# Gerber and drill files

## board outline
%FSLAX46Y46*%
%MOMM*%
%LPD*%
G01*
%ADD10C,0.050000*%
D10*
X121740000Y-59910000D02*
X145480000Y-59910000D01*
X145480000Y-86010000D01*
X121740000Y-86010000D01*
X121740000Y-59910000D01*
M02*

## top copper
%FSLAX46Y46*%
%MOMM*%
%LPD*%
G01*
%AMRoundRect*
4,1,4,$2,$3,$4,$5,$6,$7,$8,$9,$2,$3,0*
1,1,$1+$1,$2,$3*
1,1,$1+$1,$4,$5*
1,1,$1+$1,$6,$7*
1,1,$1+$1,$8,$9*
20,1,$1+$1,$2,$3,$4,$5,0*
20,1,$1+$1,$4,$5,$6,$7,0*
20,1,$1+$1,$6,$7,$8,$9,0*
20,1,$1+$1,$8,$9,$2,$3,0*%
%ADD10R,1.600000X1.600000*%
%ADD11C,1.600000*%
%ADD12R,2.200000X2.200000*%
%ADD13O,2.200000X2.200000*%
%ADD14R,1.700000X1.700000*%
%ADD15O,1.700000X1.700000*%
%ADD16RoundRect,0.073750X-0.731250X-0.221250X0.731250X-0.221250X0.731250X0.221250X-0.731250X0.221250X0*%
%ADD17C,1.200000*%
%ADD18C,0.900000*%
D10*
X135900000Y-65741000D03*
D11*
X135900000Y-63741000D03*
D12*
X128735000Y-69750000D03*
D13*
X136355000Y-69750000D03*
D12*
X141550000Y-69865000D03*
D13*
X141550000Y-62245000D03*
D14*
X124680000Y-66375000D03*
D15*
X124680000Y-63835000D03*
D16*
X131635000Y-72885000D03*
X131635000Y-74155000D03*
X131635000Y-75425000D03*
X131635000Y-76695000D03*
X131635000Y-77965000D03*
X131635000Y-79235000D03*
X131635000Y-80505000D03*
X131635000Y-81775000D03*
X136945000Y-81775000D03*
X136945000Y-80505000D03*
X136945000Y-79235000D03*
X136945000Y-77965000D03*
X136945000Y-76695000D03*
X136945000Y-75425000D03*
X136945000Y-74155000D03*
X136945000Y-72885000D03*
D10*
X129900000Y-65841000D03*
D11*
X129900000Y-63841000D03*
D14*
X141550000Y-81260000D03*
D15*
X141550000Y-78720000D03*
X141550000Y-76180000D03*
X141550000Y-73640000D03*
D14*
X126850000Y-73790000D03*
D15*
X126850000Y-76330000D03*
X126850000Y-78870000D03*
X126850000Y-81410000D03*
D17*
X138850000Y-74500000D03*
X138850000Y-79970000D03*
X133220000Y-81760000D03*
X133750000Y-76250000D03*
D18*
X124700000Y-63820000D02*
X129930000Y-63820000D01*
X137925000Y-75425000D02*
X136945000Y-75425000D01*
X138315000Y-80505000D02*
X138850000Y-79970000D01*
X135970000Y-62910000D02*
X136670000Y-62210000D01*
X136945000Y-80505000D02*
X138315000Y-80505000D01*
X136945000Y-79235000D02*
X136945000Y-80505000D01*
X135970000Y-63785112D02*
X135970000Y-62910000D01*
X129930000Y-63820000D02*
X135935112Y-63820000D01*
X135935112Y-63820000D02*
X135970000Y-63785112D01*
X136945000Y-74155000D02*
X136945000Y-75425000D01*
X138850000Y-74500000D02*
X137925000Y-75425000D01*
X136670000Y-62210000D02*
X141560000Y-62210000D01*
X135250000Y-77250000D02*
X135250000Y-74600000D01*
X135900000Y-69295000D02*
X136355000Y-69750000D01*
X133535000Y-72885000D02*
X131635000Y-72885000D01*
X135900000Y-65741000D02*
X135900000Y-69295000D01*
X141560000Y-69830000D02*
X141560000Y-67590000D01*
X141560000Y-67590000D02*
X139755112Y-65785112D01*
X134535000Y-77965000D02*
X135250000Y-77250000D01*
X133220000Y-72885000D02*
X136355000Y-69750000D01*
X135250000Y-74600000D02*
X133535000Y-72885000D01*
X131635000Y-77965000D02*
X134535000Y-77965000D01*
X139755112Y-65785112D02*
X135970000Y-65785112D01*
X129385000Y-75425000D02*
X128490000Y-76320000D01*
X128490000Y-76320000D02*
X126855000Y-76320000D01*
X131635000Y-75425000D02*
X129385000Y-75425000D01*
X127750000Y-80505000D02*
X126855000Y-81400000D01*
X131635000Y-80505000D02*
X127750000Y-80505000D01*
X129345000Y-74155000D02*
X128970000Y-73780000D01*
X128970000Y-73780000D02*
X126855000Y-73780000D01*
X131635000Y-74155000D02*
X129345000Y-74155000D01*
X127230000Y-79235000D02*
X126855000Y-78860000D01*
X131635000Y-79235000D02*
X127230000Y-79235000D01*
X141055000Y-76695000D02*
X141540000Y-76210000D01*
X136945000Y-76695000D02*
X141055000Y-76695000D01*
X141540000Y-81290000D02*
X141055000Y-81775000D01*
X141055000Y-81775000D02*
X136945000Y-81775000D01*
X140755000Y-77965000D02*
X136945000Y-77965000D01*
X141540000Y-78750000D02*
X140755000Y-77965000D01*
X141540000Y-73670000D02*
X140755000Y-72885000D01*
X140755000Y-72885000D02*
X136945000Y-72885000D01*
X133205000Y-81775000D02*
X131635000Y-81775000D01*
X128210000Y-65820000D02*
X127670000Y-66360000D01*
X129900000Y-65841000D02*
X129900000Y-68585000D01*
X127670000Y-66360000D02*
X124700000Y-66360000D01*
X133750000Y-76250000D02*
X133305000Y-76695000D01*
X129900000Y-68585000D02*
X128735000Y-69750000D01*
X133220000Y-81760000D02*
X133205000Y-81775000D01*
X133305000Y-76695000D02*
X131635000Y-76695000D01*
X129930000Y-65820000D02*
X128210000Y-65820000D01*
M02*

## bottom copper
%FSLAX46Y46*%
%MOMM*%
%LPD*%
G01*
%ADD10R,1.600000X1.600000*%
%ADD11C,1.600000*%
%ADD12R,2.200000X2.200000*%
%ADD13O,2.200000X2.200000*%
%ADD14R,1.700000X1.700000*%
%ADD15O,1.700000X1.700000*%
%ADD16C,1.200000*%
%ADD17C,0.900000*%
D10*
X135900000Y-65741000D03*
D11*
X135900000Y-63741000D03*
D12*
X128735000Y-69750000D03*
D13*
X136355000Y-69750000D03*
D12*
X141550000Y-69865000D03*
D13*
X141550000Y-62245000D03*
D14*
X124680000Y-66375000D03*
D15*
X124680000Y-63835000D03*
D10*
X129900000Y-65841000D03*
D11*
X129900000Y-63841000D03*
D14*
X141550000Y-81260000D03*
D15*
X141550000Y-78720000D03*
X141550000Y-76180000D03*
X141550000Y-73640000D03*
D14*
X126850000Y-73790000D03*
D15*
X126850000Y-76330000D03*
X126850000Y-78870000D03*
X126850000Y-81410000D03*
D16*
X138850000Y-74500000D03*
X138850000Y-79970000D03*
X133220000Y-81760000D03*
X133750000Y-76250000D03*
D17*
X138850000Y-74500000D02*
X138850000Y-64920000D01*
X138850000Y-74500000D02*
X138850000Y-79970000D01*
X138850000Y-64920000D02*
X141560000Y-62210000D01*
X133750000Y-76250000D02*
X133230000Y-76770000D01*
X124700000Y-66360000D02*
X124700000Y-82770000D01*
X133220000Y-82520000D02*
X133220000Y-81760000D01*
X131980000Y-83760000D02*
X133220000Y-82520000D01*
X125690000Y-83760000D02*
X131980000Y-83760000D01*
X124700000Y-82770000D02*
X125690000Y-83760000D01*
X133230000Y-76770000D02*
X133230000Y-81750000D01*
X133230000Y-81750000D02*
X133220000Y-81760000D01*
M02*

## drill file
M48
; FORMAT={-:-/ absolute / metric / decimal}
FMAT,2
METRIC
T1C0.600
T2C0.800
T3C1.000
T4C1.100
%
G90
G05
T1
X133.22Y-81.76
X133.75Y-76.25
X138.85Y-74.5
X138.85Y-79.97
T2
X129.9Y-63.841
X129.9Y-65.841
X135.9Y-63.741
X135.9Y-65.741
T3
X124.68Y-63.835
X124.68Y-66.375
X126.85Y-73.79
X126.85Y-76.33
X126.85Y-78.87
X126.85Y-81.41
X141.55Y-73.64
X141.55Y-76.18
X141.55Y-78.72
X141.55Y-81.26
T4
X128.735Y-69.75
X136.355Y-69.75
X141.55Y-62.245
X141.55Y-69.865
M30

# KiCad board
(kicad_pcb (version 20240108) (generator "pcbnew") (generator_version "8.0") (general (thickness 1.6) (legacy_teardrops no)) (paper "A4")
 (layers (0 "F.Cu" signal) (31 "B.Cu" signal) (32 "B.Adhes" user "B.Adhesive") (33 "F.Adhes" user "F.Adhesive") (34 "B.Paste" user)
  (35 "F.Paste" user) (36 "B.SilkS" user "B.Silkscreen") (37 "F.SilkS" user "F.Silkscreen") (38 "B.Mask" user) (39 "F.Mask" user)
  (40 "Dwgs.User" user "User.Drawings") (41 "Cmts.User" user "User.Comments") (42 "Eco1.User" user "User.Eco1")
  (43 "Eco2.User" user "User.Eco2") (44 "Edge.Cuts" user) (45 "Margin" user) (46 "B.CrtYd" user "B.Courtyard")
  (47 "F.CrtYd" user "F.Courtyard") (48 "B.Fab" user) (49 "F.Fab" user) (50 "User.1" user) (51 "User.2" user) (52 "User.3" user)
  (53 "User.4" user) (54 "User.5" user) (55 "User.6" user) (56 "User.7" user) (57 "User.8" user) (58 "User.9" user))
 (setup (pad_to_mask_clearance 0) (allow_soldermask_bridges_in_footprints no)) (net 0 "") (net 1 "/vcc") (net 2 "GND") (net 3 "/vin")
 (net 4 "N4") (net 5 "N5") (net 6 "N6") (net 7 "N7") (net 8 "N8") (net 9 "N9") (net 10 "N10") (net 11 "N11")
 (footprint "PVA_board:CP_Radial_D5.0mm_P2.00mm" (layer "F.Cu") (at 135.9 64.7 90)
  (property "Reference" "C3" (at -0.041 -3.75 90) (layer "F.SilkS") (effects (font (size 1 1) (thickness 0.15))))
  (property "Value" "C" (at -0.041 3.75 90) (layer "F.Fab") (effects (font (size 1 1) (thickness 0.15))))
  (pad "1" thru_hole rect (at -1.041 0 90) (size 1.6 1.6) (drill 0.8) (layers "*.Cu" "*.Mask") (remove_unused_layers no) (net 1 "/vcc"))
  (pad "2" thru_hole circle (at 0.959 0 90) (size 1.6 1.6) (drill 0.8) (layers "*.Cu" "*.Mask") (remove_unused_layers no) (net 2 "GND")))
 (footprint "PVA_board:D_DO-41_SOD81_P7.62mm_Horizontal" (layer "F.Cu") (at 132.5 69.75)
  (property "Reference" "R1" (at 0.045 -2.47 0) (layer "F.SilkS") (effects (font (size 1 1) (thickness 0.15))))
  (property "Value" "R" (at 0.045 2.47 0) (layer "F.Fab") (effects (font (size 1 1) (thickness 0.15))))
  (pad "1" thru_hole rect (at -3.765 0) (size 2.2 2.2) (drill 1.1) (layers "*.Cu" "*.Mask") (remove_unused_layers no) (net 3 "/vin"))
  (pad "2" thru_hole oval (at 3.855 0) (size 2.2 2.2) (drill 1.1) (layers "*.Cu" "*.Mask") (remove_unused_layers no) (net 1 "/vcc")))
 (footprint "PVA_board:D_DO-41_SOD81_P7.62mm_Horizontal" (layer "F.Cu") (at 141.55 66.1 90)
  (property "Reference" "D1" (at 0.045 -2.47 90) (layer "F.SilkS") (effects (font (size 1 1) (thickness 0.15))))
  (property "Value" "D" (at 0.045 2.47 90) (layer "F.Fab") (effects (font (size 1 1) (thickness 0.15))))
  (pad "1" thru_hole rect (at -3.765 0 90) (size 2.2 2.2) (drill 1.1) (layers "*.Cu" "*.Mask") (remove_unused_layers no) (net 1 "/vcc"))
  (pad "2" thru_hole oval (at 3.855 0 90) (size 2.2 2.2) (drill 1.1) (layers "*.Cu" "*.Mask") (remove_unused_layers no) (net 2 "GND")))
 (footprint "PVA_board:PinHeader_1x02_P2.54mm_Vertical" (layer "F.Cu") (at 124.6 65.055 180)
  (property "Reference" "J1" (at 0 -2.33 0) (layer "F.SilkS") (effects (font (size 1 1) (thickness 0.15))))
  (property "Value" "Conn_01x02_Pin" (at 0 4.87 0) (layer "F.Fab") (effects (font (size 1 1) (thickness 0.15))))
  (pad "1" thru_hole rect (at -0.08 -1.32 180) (size 1.7 1.7) (drill 1) (layers "*.Cu" "*.Mask") (remove_unused_layers no) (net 3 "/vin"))
  (pad "2" thru_hole oval (at -0.08 1.22 180) (size 1.7 1.7) (drill 1) (layers "*.Cu" "*.Mask") (remove_unused_layers no) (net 2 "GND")))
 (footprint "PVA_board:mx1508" (layer "F.Cu") (at 134.29 77.33)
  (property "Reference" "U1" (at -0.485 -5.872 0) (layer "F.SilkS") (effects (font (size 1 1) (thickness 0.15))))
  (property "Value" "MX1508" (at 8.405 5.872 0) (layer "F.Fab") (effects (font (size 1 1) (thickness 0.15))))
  (pad "1" smd roundrect (at -2.655 -4.445) (size 1.61 0.59) (layers "F.Cu" "F.Paste" "F.Mask") (roundrect_rratio 0.125) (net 1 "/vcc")
   (solder_mask_margin 0.102))
  (pad "2" smd roundrect (at -2.655 -3.175) (size 1.61 0.59) (layers "F.Cu" "F.Paste" "F.Mask") (roundrect_rratio 0.125) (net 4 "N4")
   (solder_mask_margin 0.102))
  (pad "3" smd roundrect (at -2.655 -1.905) (size 1.61 0.59) (layers "F.Cu" "F.Paste" "F.Mask") (roundrect_rratio 0.125) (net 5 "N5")
   (solder_mask_margin 0.102))
  (pad "4" smd roundrect (at -2.655 -0.635) (size 1.61 0.59) (layers "F.Cu" "F.Paste" "F.Mask") (roundrect_rratio 0.125) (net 3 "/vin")
   (solder_mask_margin 0.102))
  (pad "5" smd roundrect (at -2.655 0.635) (size 1.61 0.59) (layers "F.Cu" "F.Paste" "F.Mask") (roundrect_rratio 0.125) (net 1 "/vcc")
   (solder_mask_margin 0.102))
  (pad "6" smd roundrect (at -2.655 1.905) (size 1.61 0.59) (layers "F.Cu" "F.Paste" "F.Mask") (roundrect_rratio 0.125) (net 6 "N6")
   (solder_mask_margin 0.102))
  (pad "7" smd roundrect (at -2.655 3.175) (size 1.61 0.59) (layers "F.Cu" "F.Paste" "F.Mask") (roundrect_rratio 0.125) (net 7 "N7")
   (solder_mask_margin 0.102))
  (pad "8" smd roundrect (at -2.655 4.445) (size 1.61 0.59) (layers "F.Cu" "F.Paste" "F.Mask") (roundrect_rratio 0.125) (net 3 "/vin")
   (solder_mask_margin 0.102))
  (pad "9" smd roundrect (at 2.655 4.445) (size 1.61 0.59) (layers "F.Cu" "F.Paste" "F.Mask") (roundrect_rratio 0.125) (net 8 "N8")
   (solder_mask_margin 0.102))
  (pad "10" smd roundrect (at 2.655 3.175) (size 1.61 0.59) (layers "F.Cu" "F.Paste" "F.Mask") (roundrect_rratio 0.125) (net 2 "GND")
   (solder_mask_margin 0.102))
  (pad "11" smd roundrect (at 2.655 1.905) (size 1.61 0.59) (layers "F.Cu" "F.Paste" "F.Mask") (roundrect_rratio 0.125) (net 2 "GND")
   (solder_mask_margin 0.102))
  (pad "12" smd roundrect (at 2.655 0.635) (size 1.61 0.59) (layers "F.Cu" "F.Paste" "F.Mask") (roundrect_rratio 0.125) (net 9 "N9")
   (solder_mask_margin 0.102))
  (pad "13" smd roundrect (at 2.655 -0.635) (size 1.61 0.59) (layers "F.Cu" "F.Paste" "F.Mask") (roundrect_rratio 0.125) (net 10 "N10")
   (solder_mask_margin 0.102))
  (pad "14" smd roundrect (at 2.655 -1.905) (size 1.61 0.59) (layers "F.Cu" "F.Paste" "F.Mask") (roundrect_rratio 0.125) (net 2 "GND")
   (solder_mask_margin 0.102))
  (pad "15" smd roundrect (at 2.655 -3.175) (size 1.61 0.59) (layers "F.Cu" "F.Paste" "F.Mask") (roundrect_rratio 0.125) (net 2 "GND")
   (solder_mask_margin 0.102))
  (pad "16" smd roundrect (at 2.655 -4.445) (size 1.61 0.59) (layers "F.Cu" "F.Paste" "F.Mask") (roundrect_rratio 0.125) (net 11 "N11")
   (solder_mask_margin 0.102)))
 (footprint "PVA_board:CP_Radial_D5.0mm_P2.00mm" (layer "F.Cu") (at 129.9 64.8 90)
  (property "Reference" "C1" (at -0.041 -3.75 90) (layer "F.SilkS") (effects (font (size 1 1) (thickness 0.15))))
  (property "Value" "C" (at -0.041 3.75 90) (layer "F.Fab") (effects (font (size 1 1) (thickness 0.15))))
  (pad "1" thru_hole rect (at -1.041 0 90) (size 1.6 1.6) (drill 0.8) (layers "*.Cu" "*.Mask") (remove_unused_layers no) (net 3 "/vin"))
  (pad "2" thru_hole circle (at 0.959 0 90) (size 1.6 1.6) (drill 0.8) (layers "*.Cu" "*.Mask") (remove_unused_layers no) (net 2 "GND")))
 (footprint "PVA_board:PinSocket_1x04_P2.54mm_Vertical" (layer "F.Cu") (at 141.55 77.4 180)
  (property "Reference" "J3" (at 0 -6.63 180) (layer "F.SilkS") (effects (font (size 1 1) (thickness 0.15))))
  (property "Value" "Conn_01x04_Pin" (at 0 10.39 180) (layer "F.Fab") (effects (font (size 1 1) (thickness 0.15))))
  (pad "1" thru_hole rect (at 0 -3.86 180) (size 1.7 1.7) (drill 1) (layers "*.Cu" "*.Mask") (remove_unused_layers no) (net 8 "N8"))
  (pad "2" thru_hole oval (at 0 -1.32 180) (size 1.7 1.7) (drill 1) (layers "*.Cu" "*.Mask") (remove_unused_layers no) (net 9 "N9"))
  (pad "3" thru_hole oval (at 0 1.22 180) (size 1.7 1.7) (drill 1) (layers "*.Cu" "*.Mask") (remove_unused_layers no) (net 10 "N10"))
  (pad "4" thru_hole oval (at 0 3.76 180) (size 1.7 1.7) (drill 1) (layers "*.Cu" "*.Mask") (remove_unused_layers no) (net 11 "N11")))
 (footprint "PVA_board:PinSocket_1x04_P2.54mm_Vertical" (layer "F.Cu") (at 126.85 77.65)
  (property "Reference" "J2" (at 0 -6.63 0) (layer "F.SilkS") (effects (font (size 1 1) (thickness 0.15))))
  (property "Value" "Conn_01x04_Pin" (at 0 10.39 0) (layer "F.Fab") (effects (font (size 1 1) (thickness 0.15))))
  (pad "1" thru_hole rect (at 0 -3.86) (size 1.7 1.7) (drill 1) (layers "*.Cu" "*.Mask") (remove_unused_layers no) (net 4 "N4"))
  (pad "2" thru_hole oval (at 0 -1.32) (size 1.7 1.7) (drill 1) (layers "*.Cu" "*.Mask") (remove_unused_layers no) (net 5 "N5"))
  (pad "3" thru_hole oval (at 0 1.22) (size 1.7 1.7) (drill 1) (layers "*.Cu" "*.Mask") (remove_unused_layers no) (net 6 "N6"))
  (pad "4" thru_hole oval (at 0 3.76) (size 1.7 1.7) (drill 1) (layers "*.Cu" "*.Mask") (remove_unused_layers no) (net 7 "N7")))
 (gr_rect (start 121.74 59.91) (end 145.48 86.01) (stroke (width 0.05) (type default)) (fill none) (layer "Edge.Cuts"))
 (segment (start 124.7 63.82) (end 129.93 63.82) (width 0.9) (layer "F.Cu") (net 2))
 (segment (start 137.925 75.425) (end 136.945 75.425) (width 0.9) (layer "F.Cu") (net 2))
 (segment (start 138.315 80.505) (end 138.85 79.97) (width 0.9) (layer "F.Cu") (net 2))
 (segment (start 135.97 62.91) (end 136.67 62.21) (width 0.9) (layer "F.Cu") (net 2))
 (segment (start 136.945 80.505) (end 138.315 80.505) (width 0.9) (layer "F.Cu") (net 2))
 (segment (start 136.945 79.235) (end 136.945 80.505) (width 0.9) (layer "F.Cu") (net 2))
 (segment (start 135.97 63.785112) (end 135.97 62.91) (width 0.9) (layer "F.Cu") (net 2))
 (segment (start 129.93 63.82) (end 135.935112 63.82) (width 0.9) (layer "F.Cu") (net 2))
 (segment (start 135.935112 63.82) (end 135.97 63.785112) (width 0.9) (layer "F.Cu") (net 2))
 (segment (start 136.945 74.155) (end 136.945 75.425) (width 0.9) (layer "F.Cu") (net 2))
 (segment (start 138.85 74.5) (end 137.925 75.425) (width 0.9) (layer "F.Cu") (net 2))
 (segment (start 136.67 62.21) (end 141.56 62.21) (width 0.9) (layer "F.Cu") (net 2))
 (via (at 138.85 74.5) (size 1.2) (drill 0.6) (layers "F.Cu" "B.Cu") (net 2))
 (via (at 138.85 79.97) (size 1.2) (drill 0.6) (layers "F.Cu" "B.Cu") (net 2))
 (segment (start 138.85 74.5) (end 138.85 64.92) (width 0.9) (layer "B.Cu") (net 2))
 (segment (start 138.85 74.5) (end 138.85 79.97) (width 0.9) (layer "B.Cu") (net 2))
 (segment (start 138.85 64.92) (end 141.56 62.21) (width 0.9) (layer "B.Cu") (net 2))
 (segment (start 135.25 77.25) (end 135.25 74.6) (width 0.9) (layer "F.Cu") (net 1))
 (segment (start 135.9 69.295) (end 136.355 69.75) (width 0.9) (layer "F.Cu") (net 1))
 (segment (start 133.535 72.885) (end 131.635 72.885) (width 0.9) (layer "F.Cu") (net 1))
 (segment (start 135.9 65.741) (end 135.9 69.295) (width 0.9) (layer "F.Cu") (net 1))
 (segment (start 141.56 69.83) (end 141.56 67.59) (width 0.9) (layer "F.Cu") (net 1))
 (segment (start 141.56 67.59) (end 139.755112 65.785112) (width 0.9) (layer "F.Cu") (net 1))
 (segment (start 134.535 77.965) (end 135.25 77.25) (width 0.9) (layer "F.Cu") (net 1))
 (segment (start 133.22 72.885) (end 136.355 69.75) (width 0.9) (layer "F.Cu") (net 1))
 (segment (start 135.25 74.6) (end 133.535 72.885) (width 0.9) (layer "F.Cu") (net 1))
 (segment (start 131.635 77.965) (end 134.535 77.965) (width 0.9) (layer "F.Cu") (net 1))
 (segment (start 139.755112 65.785112) (end 135.97 65.785112) (width 0.9) (layer "F.Cu") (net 1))
 (segment (start 129.385 75.425) (end 128.49 76.32) (width 0.9) (layer "F.Cu") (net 5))
 (segment (start 128.49 76.32) (end 126.855 76.32) (width 0.9) (layer "F.Cu") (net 5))
 (segment (start 131.635 75.425) (end 129.385 75.425) (width 0.9) (layer "F.Cu") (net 5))
 (segment (start 127.75 80.505) (end 126.855 81.4) (width 0.9) (layer "F.Cu") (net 7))
 (segment (start 131.635 80.505) (end 127.75 80.505) (width 0.9) (layer "F.Cu") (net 7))
 (segment (start 129.345 74.155) (end 128.97 73.78) (width 0.9) (layer "F.Cu") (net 4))
 (segment (start 128.97 73.78) (end 126.855 73.78) (width 0.9) (layer "F.Cu") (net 4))
 (segment (start 131.635 74.155) (end 129.345 74.155) (width 0.9) (layer "F.Cu") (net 4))
 (segment (start 127.23 79.235) (end 126.855 78.86) (width 0.9) (layer "F.Cu") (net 6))
 (segment (start 131.635 79.235) (end 127.23 79.235) (width 0.9) (layer "F.Cu") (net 6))
 (segment (start 141.055 76.695) (end 141.54 76.21) (width 0.9) (layer "F.Cu") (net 10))
 (segment (start 136.945 76.695) (end 141.055 76.695) (width 0.9) (layer "F.Cu") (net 10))
 (segment (start 141.54 81.29) (end 141.055 81.775) (width 0.9) (layer "F.Cu") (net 8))
 (segment (start 141.055 81.775) (end 136.945 81.775) (width 0.9) (layer "F.Cu") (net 8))
 (segment (start 140.755 77.965) (end 136.945 77.965) (width 0.9) (layer "F.Cu") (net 9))
 (segment (start 141.54 78.75) (end 140.755 77.965) (width 0.9) (layer "F.Cu") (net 9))
 (segment (start 141.54 73.67) (end 140.755 72.885) (width 0.9) (layer "F.Cu") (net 11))
 (segment (start 140.755 72.885) (end 136.945 72.885) (width 0.9) (layer "F.Cu") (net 11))
 (segment (start 133.205 81.775) (end 131.635 81.775) (width 0.9) (layer "F.Cu") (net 3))
 (segment (start 128.21 65.82) (end 127.67 66.36) (width 0.9) (layer "F.Cu") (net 3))
 (segment (start 129.9 65.841) (end 129.9 68.585) (width 0.9) (layer "F.Cu") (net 3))
 (segment (start 127.67 66.36) (end 124.7 66.36) (width 0.9) (layer "F.Cu") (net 3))
 (segment (start 133.75 76.25) (end 133.305 76.695) (width 0.9) (layer "F.Cu") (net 3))
 (segment (start 129.9 68.585) (end 128.735 69.75) (width 0.9) (layer "F.Cu") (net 3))
 (segment (start 133.22 81.76) (end 133.205 81.775) (width 0.9) (layer "F.Cu") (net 3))
 (segment (start 133.305 76.695) (end 131.635 76.695) (width 0.9) (layer "F.Cu") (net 3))
 (segment (start 129.93 65.82) (end 128.21 65.82) (width 0.9) (layer "F.Cu") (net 3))
 (via (at 133.22 81.76) (size 1.2) (drill 0.6) (layers "F.Cu" "B.Cu") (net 3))
 (via (at 133.75 76.25) (size 1.2) (drill 0.6) (layers "F.Cu" "B.Cu") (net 3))
 (segment (start 133.75 76.25) (end 133.23 76.77) (width 0.9) (layer "B.Cu") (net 3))
 (segment (start 124.7 66.36) (end 124.7 82.77) (width 0.9) (layer "B.Cu") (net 3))
 (segment (start 133.22 82.52) (end 133.22 81.76) (width 0.9) (layer "B.Cu") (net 3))
 (segment (start 131.98 83.76) (end 133.22 82.52) (width 0.9) (layer "B.Cu") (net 3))
 (segment (start 125.69 83.76) (end 131.98 83.76) (width 0.9) (layer "B.Cu") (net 3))
 (segment (start 124.7 82.77) (end 125.69 83.76) (width 0.9) (layer "B.Cu") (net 3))
 (segment (start 133.23 76.77) (end 133.23 81.75) (width 0.9) (layer "B.Cu") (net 3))
 (segment (start 133.23 81.75) (end 133.22 81.76) (width 0.9) (layer "B.Cu") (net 3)))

